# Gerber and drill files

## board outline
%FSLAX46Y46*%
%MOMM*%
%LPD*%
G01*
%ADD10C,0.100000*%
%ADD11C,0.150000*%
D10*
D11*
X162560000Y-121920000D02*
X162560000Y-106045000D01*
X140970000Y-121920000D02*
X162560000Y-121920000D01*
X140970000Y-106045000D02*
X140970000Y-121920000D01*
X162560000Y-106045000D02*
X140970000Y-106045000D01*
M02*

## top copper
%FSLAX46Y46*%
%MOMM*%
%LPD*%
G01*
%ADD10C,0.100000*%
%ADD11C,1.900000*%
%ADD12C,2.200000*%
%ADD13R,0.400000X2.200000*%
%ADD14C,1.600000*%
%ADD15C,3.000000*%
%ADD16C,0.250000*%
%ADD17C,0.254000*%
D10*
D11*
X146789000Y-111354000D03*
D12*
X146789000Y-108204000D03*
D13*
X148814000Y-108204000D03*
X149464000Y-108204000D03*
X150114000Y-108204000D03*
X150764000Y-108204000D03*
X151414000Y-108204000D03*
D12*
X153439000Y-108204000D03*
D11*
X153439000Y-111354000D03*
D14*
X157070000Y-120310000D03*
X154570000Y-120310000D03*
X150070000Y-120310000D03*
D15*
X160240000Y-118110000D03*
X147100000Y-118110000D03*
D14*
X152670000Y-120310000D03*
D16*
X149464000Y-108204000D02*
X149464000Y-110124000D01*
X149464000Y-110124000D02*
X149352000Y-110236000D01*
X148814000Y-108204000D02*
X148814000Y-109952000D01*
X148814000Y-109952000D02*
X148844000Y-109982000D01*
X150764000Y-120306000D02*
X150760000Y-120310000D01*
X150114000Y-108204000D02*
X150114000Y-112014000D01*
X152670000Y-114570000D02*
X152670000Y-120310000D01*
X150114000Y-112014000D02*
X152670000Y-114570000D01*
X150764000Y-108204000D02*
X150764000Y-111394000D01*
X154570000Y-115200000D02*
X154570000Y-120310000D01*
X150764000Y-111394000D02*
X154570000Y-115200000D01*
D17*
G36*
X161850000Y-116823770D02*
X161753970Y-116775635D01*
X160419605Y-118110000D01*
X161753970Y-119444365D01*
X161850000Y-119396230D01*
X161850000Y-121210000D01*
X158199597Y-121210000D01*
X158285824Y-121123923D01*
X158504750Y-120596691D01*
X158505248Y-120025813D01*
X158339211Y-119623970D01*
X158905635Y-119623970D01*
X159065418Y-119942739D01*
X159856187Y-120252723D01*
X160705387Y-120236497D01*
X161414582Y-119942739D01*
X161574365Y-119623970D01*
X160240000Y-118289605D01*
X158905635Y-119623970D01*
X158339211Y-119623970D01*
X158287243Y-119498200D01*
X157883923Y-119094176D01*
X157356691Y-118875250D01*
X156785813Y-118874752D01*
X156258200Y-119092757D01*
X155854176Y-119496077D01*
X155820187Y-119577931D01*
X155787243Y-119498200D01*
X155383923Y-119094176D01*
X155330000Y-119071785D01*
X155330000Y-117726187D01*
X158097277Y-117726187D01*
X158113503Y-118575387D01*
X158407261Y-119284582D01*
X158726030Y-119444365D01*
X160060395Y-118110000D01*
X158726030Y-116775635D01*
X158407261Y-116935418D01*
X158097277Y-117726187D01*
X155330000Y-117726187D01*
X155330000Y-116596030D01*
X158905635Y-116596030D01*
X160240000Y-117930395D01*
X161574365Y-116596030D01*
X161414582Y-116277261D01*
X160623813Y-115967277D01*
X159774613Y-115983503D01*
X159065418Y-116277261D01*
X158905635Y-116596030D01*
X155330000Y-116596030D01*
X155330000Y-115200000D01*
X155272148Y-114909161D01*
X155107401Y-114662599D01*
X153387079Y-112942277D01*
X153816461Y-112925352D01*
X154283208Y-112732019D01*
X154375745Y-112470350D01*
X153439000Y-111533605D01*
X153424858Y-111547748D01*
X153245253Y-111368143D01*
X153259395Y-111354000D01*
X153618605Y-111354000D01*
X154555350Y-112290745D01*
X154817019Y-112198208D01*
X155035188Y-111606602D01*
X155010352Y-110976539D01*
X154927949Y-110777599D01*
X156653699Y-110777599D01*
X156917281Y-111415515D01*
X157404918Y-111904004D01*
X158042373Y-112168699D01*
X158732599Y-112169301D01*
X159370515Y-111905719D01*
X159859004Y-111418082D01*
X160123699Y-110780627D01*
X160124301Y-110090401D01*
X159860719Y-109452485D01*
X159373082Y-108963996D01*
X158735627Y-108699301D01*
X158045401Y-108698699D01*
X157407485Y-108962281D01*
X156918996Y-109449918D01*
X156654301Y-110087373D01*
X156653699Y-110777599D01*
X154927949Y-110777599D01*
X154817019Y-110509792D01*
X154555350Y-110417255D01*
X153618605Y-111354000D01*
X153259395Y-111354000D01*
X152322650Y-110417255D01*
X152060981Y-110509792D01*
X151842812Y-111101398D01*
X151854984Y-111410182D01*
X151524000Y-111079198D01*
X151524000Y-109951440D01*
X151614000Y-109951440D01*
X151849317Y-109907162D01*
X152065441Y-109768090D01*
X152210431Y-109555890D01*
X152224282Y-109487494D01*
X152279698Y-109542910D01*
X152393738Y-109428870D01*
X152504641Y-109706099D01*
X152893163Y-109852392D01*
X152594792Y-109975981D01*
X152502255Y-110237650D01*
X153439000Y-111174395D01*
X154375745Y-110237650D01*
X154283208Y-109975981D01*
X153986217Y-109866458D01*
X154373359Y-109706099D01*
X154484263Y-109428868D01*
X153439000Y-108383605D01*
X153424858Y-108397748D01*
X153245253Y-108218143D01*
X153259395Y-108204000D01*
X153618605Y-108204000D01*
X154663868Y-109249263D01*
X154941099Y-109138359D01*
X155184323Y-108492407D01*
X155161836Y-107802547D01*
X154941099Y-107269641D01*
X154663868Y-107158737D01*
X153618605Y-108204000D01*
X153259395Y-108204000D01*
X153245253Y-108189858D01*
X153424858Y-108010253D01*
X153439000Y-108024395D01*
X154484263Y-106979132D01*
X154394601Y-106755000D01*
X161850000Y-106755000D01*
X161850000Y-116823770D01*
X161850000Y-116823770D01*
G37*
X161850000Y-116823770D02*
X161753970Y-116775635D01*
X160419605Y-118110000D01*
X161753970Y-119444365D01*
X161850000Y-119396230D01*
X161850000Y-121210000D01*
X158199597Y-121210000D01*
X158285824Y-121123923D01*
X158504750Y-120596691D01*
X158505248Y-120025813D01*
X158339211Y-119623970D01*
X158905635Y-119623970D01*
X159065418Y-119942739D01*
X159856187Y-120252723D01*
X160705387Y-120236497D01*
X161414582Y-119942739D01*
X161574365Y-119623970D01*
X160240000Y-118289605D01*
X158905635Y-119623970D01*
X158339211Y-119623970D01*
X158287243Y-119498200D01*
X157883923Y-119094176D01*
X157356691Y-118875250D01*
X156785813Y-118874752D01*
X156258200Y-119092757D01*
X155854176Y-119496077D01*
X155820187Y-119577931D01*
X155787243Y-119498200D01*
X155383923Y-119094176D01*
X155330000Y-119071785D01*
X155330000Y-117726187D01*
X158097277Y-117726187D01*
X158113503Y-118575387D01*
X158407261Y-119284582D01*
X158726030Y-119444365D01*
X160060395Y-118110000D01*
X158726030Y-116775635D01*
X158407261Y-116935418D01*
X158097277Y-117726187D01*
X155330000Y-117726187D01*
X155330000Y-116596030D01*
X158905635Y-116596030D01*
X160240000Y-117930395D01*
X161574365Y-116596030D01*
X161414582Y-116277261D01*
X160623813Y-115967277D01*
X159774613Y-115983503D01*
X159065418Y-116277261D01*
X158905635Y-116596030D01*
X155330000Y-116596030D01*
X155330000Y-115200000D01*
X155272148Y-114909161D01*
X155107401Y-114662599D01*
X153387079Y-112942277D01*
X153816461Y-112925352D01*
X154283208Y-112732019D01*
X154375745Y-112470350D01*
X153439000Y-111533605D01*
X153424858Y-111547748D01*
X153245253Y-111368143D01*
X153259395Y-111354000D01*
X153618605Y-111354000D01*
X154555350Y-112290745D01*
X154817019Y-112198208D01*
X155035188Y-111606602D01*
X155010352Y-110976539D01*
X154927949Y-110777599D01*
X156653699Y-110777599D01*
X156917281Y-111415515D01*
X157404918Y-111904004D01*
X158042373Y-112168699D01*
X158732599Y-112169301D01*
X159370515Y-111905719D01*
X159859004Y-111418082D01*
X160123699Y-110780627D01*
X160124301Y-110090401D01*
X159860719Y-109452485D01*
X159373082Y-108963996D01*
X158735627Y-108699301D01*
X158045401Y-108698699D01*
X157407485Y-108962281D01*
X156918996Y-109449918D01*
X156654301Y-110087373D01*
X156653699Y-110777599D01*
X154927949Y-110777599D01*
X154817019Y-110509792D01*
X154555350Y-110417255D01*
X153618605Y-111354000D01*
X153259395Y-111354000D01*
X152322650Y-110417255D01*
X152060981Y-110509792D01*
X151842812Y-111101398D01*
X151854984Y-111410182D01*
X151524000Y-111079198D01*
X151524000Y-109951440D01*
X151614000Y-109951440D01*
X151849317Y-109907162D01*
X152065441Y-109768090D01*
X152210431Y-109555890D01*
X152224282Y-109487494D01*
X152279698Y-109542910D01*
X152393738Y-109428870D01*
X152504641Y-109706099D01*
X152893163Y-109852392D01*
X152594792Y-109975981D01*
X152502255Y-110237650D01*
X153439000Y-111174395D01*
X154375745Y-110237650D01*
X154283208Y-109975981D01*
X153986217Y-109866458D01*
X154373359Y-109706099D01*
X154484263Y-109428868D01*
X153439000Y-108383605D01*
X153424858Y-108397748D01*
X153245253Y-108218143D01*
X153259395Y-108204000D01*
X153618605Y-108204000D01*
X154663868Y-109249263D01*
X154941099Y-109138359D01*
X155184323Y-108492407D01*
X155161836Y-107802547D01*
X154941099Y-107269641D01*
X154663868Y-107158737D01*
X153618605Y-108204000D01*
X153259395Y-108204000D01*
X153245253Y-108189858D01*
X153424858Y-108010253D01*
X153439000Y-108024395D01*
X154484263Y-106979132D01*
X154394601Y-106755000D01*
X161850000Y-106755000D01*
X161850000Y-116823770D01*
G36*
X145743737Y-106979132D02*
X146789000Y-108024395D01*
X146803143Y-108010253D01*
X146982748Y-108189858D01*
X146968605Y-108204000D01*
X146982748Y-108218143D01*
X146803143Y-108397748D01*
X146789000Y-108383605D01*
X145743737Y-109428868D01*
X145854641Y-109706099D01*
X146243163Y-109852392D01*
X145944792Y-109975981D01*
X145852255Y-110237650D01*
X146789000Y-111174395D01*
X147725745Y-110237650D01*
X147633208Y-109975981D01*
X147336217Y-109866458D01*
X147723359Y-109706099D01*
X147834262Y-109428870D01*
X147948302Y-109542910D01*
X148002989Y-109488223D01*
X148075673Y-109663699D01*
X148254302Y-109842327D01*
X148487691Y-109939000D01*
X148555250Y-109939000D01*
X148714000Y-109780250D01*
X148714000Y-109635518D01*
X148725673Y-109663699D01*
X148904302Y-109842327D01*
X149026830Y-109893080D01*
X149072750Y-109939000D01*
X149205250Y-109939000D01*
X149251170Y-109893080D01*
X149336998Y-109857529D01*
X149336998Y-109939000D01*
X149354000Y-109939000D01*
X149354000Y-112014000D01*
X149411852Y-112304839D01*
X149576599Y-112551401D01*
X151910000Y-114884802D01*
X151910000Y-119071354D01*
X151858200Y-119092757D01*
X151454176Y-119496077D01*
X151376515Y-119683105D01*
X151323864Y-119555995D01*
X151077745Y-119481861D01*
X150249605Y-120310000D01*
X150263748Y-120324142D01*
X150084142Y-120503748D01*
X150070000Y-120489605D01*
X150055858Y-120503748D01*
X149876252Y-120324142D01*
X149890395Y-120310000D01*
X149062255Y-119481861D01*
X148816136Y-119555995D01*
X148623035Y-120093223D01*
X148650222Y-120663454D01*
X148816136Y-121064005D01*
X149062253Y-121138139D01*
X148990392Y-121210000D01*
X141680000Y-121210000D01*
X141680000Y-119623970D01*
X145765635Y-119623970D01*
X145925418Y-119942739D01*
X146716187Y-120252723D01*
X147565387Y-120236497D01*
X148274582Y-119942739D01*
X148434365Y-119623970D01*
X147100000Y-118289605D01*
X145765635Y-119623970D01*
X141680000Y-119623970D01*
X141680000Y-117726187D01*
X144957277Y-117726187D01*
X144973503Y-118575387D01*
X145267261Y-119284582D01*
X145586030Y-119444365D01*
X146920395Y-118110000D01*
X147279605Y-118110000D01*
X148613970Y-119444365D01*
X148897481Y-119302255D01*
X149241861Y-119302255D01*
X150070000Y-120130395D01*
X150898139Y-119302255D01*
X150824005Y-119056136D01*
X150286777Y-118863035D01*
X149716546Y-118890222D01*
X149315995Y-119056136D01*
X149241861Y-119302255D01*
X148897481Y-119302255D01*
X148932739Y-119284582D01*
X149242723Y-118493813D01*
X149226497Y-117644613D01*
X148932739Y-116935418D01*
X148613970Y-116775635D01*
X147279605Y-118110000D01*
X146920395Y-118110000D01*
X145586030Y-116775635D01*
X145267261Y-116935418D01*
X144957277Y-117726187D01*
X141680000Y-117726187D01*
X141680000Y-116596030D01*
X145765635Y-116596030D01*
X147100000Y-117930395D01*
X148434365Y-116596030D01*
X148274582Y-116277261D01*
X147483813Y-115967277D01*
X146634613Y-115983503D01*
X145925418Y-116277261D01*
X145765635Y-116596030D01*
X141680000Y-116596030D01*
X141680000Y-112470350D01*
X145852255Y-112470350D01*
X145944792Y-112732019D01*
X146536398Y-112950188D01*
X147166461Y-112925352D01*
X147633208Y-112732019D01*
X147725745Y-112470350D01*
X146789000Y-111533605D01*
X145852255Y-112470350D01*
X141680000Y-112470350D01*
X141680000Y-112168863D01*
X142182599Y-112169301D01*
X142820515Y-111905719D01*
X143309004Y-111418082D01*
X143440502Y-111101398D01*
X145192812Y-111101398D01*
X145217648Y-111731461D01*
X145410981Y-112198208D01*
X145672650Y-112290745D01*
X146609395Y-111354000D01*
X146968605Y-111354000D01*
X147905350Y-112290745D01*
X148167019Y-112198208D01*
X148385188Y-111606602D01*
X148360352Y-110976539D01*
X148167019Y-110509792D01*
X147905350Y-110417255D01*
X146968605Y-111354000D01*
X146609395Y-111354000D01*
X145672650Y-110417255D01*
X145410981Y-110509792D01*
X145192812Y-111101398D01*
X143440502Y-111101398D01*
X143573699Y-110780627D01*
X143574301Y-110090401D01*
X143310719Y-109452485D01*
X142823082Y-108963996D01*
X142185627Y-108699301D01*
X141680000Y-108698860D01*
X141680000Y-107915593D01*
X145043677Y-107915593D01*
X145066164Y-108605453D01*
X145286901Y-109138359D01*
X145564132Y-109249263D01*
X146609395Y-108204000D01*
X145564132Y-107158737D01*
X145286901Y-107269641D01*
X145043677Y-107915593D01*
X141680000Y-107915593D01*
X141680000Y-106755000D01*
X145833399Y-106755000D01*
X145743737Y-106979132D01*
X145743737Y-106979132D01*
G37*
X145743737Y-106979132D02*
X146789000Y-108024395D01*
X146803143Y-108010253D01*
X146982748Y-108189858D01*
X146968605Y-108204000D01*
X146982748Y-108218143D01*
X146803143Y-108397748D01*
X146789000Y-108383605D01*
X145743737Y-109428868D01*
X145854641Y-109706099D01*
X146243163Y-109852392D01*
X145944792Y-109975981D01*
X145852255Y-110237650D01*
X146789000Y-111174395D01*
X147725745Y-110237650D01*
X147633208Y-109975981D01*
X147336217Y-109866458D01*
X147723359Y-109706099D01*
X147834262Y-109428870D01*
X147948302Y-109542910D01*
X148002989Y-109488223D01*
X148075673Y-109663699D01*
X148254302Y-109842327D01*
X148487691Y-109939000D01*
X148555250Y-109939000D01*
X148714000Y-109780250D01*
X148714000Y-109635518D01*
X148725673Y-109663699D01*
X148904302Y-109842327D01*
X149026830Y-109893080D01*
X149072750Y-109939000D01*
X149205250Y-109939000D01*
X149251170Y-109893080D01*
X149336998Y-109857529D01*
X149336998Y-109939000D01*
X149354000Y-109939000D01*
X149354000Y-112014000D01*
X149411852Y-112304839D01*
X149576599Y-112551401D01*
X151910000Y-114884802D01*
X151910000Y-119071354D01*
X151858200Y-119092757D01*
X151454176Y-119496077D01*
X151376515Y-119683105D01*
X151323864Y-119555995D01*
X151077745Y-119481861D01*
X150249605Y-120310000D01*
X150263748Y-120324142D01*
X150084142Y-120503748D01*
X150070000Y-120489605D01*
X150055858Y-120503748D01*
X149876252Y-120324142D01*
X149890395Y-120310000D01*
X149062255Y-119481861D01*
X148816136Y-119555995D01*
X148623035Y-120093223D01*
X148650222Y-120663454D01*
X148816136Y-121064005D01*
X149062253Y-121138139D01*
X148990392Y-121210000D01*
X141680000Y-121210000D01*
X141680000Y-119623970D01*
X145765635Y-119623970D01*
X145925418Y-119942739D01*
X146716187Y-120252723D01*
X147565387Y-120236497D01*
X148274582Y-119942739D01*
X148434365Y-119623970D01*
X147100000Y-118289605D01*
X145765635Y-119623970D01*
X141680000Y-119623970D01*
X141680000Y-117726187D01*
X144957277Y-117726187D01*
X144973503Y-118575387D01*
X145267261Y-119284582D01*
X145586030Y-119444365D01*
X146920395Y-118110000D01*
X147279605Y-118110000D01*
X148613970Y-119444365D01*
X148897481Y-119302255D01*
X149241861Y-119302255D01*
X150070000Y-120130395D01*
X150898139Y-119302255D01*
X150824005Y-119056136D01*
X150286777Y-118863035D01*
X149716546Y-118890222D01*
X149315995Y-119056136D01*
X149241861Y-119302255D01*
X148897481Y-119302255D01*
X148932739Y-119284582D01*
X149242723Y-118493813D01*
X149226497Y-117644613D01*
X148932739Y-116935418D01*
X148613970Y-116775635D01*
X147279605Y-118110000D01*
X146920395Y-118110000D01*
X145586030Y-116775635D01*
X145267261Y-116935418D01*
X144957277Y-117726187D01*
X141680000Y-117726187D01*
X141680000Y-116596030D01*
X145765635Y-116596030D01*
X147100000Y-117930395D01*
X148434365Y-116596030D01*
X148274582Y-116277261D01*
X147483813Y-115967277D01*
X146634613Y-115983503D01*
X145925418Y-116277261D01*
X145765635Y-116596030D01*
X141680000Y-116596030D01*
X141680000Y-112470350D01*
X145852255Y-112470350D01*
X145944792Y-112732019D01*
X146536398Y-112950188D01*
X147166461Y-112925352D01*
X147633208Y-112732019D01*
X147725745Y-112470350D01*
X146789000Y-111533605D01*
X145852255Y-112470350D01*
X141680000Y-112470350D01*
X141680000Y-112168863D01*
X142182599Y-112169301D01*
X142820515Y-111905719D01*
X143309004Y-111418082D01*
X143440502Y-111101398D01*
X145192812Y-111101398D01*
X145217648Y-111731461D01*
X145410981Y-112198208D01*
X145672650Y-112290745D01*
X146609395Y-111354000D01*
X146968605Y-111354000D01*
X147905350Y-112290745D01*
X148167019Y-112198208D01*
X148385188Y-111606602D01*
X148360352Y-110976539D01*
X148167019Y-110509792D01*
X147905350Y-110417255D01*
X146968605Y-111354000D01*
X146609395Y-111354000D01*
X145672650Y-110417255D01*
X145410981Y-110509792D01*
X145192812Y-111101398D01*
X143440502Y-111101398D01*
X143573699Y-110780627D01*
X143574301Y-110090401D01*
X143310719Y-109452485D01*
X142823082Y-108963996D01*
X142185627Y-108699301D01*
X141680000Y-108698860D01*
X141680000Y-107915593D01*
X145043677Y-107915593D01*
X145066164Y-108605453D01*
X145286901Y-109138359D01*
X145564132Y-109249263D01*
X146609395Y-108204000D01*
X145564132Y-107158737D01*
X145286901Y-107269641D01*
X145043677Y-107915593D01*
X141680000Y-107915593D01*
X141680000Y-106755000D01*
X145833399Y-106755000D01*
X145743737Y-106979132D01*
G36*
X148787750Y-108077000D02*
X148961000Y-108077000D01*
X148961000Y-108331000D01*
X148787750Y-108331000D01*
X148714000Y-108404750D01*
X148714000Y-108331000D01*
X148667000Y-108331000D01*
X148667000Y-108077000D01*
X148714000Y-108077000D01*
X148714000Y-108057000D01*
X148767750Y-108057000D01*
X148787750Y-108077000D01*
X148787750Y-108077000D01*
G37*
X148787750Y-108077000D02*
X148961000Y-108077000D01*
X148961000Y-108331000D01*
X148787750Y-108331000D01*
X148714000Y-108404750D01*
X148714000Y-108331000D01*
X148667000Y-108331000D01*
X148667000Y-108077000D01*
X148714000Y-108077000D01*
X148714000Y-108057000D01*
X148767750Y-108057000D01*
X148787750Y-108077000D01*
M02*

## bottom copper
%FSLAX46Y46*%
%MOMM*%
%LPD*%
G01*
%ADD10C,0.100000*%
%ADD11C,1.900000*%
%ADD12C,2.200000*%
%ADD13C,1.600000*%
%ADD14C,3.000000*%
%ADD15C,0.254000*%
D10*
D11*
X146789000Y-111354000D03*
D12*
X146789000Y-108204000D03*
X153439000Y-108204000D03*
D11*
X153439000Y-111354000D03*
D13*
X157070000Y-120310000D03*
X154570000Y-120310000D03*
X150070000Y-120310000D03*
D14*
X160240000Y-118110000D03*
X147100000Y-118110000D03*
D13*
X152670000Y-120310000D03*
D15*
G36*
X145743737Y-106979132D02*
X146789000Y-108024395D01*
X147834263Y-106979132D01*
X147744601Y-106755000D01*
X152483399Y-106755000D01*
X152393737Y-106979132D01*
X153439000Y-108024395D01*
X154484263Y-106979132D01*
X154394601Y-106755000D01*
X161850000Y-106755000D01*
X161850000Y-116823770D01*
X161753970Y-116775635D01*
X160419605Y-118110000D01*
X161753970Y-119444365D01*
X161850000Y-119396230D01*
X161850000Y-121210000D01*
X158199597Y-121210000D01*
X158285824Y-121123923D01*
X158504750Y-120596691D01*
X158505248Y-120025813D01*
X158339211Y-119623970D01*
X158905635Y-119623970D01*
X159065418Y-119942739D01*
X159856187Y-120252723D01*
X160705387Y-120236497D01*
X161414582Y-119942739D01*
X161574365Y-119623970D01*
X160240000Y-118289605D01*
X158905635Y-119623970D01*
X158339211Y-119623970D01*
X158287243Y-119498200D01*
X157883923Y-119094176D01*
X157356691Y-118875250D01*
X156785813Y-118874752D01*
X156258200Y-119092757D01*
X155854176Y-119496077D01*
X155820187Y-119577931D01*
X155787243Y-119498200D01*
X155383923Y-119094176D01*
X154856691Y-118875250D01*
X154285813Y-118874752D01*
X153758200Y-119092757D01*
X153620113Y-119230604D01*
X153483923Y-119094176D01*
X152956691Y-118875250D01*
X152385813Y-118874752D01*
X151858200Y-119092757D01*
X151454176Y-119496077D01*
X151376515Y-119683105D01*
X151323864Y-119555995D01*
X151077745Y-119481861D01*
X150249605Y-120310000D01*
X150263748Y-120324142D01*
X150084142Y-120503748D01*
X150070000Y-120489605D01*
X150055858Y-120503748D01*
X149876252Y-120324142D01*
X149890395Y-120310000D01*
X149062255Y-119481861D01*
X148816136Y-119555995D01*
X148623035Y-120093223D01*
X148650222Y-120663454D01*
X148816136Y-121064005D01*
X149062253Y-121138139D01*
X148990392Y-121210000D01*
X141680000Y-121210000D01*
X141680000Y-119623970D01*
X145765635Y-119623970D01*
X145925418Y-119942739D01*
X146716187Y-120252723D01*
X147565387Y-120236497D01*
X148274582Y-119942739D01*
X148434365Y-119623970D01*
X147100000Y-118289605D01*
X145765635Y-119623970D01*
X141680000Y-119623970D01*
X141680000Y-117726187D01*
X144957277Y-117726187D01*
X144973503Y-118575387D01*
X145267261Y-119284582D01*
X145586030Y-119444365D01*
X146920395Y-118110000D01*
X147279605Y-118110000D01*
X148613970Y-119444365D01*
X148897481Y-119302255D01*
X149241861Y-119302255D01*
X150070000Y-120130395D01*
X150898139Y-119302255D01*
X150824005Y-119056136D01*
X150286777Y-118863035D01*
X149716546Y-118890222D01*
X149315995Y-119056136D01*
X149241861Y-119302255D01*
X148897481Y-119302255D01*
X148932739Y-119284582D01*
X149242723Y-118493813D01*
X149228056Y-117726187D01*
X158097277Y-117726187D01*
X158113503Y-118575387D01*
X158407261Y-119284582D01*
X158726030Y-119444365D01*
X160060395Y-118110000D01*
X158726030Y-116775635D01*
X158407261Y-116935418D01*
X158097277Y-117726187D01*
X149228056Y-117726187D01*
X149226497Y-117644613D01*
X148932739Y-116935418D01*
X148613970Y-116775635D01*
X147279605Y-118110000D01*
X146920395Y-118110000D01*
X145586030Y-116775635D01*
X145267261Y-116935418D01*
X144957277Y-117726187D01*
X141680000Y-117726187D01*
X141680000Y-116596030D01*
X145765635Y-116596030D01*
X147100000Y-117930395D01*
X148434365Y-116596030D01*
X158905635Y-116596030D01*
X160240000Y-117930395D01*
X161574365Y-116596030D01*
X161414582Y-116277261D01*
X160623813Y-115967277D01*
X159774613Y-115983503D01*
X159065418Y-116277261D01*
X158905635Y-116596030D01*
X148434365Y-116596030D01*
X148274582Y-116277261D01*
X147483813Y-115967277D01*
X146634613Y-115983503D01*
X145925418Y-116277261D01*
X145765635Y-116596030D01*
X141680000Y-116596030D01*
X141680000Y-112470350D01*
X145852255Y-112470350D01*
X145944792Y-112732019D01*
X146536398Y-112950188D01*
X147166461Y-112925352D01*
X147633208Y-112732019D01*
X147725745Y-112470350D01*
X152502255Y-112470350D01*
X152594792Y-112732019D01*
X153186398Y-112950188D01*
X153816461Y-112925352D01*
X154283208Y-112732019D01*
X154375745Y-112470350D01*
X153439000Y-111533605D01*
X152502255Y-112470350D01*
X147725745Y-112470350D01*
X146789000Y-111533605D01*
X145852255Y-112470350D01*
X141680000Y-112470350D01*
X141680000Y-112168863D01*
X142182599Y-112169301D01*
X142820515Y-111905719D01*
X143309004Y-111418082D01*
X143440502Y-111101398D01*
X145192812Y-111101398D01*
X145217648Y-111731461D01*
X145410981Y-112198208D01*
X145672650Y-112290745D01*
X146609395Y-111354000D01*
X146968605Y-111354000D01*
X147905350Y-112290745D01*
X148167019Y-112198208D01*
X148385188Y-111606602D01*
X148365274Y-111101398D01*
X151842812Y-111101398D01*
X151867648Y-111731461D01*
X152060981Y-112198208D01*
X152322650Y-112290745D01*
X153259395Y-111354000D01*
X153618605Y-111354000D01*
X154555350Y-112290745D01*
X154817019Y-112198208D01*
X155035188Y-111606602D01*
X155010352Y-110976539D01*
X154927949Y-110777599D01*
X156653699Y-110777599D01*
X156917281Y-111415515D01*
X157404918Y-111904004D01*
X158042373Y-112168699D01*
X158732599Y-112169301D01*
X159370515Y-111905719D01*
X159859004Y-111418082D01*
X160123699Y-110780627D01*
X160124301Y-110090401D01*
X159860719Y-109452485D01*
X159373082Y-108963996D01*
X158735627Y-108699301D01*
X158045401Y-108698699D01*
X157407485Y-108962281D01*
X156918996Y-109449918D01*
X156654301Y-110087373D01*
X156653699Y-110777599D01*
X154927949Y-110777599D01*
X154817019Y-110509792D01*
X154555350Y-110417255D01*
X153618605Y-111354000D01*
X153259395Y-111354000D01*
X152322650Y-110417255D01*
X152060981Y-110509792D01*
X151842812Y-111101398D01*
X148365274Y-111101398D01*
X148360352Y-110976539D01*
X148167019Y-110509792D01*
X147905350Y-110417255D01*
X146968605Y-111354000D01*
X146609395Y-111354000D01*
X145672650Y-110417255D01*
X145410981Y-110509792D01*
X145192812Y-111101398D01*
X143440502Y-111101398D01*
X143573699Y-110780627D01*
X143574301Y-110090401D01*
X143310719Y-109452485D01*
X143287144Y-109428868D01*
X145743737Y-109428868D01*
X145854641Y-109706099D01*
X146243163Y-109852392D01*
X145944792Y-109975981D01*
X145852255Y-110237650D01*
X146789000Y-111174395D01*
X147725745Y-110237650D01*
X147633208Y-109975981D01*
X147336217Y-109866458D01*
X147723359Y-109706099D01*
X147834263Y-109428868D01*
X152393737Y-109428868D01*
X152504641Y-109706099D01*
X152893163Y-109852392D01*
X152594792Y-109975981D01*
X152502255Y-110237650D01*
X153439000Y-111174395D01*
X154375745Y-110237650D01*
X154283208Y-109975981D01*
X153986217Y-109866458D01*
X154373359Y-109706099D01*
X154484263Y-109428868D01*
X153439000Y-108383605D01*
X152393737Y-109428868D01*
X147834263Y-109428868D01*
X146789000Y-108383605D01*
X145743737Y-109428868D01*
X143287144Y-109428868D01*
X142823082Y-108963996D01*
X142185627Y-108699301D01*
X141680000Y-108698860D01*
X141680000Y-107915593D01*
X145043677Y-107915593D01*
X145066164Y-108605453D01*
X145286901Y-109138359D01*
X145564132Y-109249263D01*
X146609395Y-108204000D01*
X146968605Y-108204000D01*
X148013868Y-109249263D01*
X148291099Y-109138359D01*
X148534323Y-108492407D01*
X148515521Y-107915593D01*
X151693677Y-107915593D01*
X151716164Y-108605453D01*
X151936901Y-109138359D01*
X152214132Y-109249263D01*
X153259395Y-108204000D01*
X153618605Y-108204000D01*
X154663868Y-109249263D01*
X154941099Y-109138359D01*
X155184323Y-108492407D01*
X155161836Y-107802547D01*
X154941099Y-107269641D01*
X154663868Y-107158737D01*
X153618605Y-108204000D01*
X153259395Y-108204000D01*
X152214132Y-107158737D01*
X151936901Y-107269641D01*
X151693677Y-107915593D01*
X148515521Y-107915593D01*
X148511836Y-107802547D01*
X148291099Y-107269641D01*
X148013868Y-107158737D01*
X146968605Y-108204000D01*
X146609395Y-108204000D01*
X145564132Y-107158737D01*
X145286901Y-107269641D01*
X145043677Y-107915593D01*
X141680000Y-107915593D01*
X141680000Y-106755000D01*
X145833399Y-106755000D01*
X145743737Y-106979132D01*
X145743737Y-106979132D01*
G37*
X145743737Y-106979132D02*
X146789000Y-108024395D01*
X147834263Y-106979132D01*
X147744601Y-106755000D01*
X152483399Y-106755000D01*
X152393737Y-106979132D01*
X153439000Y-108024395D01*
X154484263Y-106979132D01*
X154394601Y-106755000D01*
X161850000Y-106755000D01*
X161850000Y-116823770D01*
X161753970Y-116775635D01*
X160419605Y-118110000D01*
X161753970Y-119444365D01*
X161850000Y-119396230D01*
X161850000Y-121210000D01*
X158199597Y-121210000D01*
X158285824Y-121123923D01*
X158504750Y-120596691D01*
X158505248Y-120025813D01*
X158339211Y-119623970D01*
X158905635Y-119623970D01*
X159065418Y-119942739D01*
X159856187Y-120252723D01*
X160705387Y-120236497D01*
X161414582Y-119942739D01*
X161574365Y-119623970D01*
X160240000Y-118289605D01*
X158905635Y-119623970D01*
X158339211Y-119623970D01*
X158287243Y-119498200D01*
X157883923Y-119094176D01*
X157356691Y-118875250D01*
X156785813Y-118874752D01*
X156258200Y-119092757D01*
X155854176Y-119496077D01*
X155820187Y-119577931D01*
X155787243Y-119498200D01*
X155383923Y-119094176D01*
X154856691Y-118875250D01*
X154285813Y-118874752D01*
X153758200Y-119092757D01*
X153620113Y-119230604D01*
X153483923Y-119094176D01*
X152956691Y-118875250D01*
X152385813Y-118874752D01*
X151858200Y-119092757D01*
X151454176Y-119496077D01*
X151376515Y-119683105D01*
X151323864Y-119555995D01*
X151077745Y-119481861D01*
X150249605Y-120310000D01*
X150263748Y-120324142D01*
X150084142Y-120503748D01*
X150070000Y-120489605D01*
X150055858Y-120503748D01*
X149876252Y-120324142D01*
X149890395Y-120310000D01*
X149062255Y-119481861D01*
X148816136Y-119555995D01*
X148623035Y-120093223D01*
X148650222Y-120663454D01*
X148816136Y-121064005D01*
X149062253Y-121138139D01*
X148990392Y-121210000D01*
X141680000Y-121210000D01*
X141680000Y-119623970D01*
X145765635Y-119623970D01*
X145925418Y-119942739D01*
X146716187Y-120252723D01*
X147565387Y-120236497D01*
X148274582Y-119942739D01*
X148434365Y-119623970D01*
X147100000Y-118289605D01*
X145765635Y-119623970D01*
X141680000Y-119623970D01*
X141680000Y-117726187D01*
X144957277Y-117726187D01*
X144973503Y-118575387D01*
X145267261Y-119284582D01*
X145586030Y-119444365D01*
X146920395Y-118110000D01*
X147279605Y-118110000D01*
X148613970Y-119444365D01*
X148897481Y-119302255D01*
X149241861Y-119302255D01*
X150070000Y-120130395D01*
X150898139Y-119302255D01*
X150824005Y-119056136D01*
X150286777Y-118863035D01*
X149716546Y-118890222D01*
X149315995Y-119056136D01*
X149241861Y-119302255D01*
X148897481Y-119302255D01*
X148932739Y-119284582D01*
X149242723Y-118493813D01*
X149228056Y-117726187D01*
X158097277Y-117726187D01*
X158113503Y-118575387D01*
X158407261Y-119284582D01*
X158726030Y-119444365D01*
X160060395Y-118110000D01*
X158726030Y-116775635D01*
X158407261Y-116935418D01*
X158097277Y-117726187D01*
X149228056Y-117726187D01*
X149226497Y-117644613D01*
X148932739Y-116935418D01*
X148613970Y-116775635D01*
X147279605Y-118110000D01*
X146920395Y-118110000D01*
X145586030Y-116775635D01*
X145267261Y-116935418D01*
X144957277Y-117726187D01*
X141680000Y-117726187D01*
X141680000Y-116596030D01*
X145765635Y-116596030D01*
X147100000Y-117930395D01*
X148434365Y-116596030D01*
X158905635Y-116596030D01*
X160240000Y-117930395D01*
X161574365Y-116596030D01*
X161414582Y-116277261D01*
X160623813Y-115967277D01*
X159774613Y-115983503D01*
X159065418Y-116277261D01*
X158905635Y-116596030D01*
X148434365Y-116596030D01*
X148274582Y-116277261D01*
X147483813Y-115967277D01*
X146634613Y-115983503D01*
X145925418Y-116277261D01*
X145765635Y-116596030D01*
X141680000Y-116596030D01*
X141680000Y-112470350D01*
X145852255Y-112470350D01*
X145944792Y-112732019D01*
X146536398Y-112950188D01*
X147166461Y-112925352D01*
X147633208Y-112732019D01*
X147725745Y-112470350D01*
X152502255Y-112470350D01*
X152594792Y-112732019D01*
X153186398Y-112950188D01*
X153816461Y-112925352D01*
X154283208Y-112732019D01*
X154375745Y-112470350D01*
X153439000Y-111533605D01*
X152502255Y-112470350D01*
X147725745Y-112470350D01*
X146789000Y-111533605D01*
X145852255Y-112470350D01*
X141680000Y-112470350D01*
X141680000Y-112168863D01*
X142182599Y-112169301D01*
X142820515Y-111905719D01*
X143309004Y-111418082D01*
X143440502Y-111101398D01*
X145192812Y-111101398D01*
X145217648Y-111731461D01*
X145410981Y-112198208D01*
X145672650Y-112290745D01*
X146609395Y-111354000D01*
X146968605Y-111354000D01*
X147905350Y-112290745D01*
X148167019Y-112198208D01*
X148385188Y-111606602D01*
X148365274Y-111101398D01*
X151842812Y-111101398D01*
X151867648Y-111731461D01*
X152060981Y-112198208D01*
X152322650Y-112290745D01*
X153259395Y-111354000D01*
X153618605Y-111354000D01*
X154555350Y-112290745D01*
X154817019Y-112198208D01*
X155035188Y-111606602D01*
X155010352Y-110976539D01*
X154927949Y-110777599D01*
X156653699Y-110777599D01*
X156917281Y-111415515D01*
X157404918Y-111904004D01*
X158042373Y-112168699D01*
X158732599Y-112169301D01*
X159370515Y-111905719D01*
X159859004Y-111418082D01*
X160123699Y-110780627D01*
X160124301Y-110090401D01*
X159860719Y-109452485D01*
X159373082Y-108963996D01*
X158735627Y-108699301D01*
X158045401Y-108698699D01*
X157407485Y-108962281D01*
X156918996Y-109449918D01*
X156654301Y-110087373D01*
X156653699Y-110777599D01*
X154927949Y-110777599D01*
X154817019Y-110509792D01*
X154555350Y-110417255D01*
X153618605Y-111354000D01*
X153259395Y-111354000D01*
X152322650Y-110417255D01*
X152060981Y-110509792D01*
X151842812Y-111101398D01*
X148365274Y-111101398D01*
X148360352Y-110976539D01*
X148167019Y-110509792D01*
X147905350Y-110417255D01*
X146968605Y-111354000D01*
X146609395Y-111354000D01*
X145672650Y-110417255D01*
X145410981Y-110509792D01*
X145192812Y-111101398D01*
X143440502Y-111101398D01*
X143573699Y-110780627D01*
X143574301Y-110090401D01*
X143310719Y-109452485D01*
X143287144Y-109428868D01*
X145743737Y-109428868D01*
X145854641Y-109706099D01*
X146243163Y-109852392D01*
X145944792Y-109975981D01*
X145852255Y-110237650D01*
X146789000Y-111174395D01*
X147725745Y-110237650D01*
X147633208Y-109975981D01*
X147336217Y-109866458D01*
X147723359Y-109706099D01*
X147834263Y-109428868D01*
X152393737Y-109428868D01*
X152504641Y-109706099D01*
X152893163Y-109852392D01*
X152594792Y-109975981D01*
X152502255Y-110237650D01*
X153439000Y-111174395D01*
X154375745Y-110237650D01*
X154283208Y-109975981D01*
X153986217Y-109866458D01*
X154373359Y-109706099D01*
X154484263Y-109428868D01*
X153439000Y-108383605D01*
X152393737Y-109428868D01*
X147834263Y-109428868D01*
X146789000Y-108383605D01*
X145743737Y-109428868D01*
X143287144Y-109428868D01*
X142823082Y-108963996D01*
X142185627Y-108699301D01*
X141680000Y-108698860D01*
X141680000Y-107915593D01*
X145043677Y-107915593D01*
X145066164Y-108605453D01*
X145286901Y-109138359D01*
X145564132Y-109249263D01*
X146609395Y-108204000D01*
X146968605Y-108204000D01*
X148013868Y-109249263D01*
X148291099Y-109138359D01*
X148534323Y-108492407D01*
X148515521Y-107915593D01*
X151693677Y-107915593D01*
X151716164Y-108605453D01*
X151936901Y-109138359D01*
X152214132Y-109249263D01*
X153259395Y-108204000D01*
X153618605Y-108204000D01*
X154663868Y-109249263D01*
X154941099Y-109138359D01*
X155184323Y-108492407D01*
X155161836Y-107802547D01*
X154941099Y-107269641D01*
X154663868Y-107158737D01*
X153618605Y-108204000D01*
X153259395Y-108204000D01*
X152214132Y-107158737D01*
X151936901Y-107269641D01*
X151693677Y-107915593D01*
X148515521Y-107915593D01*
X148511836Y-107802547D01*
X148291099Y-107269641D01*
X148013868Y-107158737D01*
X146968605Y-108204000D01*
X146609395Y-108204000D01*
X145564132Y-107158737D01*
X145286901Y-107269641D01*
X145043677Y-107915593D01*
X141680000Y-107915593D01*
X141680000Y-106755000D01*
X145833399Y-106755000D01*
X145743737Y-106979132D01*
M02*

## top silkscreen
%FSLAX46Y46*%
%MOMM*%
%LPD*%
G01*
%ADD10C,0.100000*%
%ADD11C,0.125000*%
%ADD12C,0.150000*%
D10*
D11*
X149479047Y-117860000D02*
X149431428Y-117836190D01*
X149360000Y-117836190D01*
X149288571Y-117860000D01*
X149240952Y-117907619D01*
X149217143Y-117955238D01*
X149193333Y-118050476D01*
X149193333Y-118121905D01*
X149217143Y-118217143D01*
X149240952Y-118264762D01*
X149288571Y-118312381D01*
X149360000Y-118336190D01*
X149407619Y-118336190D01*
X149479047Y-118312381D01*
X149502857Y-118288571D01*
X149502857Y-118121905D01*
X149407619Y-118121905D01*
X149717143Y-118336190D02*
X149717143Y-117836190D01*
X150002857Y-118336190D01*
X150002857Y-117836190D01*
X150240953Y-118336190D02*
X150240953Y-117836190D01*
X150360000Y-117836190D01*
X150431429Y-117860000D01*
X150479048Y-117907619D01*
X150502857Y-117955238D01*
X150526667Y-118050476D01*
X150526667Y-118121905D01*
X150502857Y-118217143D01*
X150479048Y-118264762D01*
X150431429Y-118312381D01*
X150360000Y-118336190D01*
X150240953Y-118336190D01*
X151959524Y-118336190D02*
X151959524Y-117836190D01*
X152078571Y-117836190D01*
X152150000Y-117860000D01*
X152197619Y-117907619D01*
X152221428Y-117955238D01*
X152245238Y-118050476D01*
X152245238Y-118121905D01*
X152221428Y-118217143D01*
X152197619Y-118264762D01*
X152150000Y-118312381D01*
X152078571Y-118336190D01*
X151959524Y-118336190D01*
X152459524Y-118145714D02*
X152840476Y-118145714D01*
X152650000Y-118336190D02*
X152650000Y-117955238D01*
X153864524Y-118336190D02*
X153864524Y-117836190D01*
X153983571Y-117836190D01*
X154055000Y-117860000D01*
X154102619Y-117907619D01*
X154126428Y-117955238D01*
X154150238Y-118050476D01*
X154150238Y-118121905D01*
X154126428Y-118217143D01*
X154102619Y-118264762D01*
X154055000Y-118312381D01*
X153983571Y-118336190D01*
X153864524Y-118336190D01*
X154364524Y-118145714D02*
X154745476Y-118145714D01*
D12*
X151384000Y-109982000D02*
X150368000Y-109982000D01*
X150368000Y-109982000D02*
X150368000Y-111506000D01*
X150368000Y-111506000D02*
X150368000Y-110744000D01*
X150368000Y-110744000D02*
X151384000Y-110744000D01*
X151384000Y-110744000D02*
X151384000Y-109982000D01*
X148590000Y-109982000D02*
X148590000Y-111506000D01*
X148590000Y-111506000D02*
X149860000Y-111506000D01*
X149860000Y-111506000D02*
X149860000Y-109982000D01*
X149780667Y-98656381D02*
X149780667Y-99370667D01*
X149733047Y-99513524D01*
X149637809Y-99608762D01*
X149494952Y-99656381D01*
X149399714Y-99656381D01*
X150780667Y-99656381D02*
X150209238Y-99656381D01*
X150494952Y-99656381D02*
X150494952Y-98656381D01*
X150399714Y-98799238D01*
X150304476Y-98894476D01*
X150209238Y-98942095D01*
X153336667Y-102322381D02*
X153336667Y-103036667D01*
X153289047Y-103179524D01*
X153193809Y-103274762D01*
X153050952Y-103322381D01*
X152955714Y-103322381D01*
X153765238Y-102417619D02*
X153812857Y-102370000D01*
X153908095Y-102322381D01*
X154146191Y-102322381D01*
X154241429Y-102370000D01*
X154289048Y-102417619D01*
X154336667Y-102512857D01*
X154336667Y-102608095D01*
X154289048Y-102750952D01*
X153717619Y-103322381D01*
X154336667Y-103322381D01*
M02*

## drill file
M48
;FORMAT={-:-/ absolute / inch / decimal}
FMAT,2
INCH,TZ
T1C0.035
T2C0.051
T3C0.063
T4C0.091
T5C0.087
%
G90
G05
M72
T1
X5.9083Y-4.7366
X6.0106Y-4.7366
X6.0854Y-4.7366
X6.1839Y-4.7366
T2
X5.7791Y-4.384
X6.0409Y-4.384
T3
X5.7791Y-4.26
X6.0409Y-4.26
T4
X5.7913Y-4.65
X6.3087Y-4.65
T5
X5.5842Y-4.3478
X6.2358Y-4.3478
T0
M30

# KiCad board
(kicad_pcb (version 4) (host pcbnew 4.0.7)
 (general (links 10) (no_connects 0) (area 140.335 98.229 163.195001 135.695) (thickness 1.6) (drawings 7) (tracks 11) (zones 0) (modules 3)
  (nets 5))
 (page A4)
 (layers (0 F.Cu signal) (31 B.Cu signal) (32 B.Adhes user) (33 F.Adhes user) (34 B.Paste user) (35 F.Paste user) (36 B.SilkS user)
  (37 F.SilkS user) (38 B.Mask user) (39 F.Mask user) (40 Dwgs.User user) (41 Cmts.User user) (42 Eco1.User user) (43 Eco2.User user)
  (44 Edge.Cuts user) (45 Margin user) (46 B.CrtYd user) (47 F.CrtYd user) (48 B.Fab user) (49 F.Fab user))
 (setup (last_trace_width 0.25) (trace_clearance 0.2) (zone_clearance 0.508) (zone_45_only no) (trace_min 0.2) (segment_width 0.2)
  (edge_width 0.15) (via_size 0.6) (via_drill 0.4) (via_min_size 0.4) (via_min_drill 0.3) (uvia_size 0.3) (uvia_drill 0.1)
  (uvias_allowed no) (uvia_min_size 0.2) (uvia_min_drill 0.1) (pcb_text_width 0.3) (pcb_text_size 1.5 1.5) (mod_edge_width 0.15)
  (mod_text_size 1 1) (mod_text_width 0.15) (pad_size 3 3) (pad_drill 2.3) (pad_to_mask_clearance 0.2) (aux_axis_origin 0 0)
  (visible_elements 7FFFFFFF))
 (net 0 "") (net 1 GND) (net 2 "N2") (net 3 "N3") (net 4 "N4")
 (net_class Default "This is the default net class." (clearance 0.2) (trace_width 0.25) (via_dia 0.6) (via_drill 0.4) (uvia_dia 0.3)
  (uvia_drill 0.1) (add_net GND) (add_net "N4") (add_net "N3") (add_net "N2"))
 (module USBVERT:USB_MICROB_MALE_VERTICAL (layer F.Cu) (at 150.114 108.204 180)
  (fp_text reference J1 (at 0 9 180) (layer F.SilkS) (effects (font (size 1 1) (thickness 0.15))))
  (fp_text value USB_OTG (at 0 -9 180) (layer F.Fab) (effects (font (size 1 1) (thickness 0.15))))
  (fp_line (start -1.27 -1.778) (end -0.254 -1.778) (layer F.SilkS) (width 0.15))
  (fp_line (start -0.254 -1.778) (end -0.254 -3.302) (layer F.SilkS) (width 0.15))
  (fp_line (start -0.254 -3.302) (end -0.254 -2.54) (layer F.SilkS) (width 0.15))
  (fp_line (start -0.254 -2.54) (end -1.27 -2.54) (layer F.SilkS) (width 0.15))
  (fp_line (start -1.27 -2.54) (end -1.27 -1.778) (layer F.SilkS) (width 0.15))
  (fp_line (start 1.524 -1.778) (end 1.524 -3.302) (layer F.SilkS) (width 0.15))
  (fp_line (start 1.524 -3.302) (end 0.254 -3.302) (layer F.SilkS) (width 0.15))
  (fp_line (start 0.254 -3.302) (end 0.254 -1.778) (layer F.SilkS) (width 0.15))
  (pad "" np_thru_hole circle (at 8.275 -2.23 180) (size 2.2 2.2) (drill 2.2) (layers *.Cu *.Mask))
  (pad 6 thru_hole circle (at 3.325 -3.15 180) (size 1.9 1.9) (drill 1.3) (layers *.Cu *.Mask) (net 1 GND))
  (pad 6 thru_hole circle (at 3.325 0 180) (size 2.2 2.2) (drill 1.6) (layers *.Cu *.Mask) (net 1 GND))
  (pad 5 smd rect (at 1.3 0 180) (size 0.4 2.2) (layers F.Cu F.Paste F.Mask) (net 1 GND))
  (pad 4 smd rect (at 0.65 0 180) (size 0.4 2.2) (layers F.Cu F.Paste F.Mask) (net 1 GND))
  (pad 3 smd rect (at 0 0 180) (size 0.4 2.2) (layers F.Cu F.Paste F.Mask) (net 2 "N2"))
  (pad 2 smd rect (at -0.65 0 180) (size 0.4 2.2) (layers F.Cu F.Paste F.Mask) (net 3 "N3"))
  (pad 1 smd rect (at -1.3 0 180) (size 0.4 2.2) (layers F.Cu F.Paste F.Mask) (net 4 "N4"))
  (pad 6 thru_hole circle (at -3.325 0 180) (size 2.2 2.2) (drill 1.6) (layers *.Cu *.Mask) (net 1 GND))
  (pad 6 thru_hole circle (at -3.325 -3.15 180) (size 1.9 1.9) (drill 1.3) (layers *.Cu *.Mask) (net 1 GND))
  (pad "" np_thru_hole circle (at -8.275 -2.23 180) (size 2.2 2.2) (drill 2.2) (layers *.Cu *.Mask)))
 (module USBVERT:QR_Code (layer B.Cu) (at 153.67 115.57)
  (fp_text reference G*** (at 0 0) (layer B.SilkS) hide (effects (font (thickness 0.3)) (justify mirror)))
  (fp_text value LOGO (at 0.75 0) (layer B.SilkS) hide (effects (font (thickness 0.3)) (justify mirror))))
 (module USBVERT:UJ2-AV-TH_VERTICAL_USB (layer F.Cu) (at 153.67 118.11 180)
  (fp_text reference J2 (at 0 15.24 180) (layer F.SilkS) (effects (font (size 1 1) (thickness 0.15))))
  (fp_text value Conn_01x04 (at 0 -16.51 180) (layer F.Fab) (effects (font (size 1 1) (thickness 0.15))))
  (pad 1 thru_hole circle (at -3.4 -2.2 180) (size 1.6 1.6) (drill 0.9) (layers *.Cu *.Mask))
  (pad 2 thru_hole circle (at -0.9 -2.2 180) (size 1.6 1.6) (drill 0.9) (layers *.Cu *.Mask) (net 3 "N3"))
  (pad 4 thru_hole circle (at 3.6 -2.2 180) (size 1.6 1.6) (drill 0.9) (layers *.Cu *.Mask) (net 1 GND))
  (pad 5 thru_hole circle (at -6.57 0 180) (size 3 3) (drill 2.3) (layers *.Cu *.Mask) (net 1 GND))
  (pad 5 thru_hole circle (at 6.57 0 180) (size 3 3) (drill 2.3) (layers *.Cu *.Mask) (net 1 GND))
  (pad 3 thru_hole circle (at 1 -2.2 180) (size 1.6 1.6) (drill 0.9) (layers *.Cu *.Mask) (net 2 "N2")))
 (gr_line (start 162.56 121.92) (end 162.56 106.045) (angle 90) (layer Edge.Cuts) (width 0.15))
 (gr_line (start 140.97 121.92) (end 162.56 121.92) (angle 90) (layer Edge.Cuts) (width 0.15))
 (gr_line (start 140.97 106.045) (end 140.97 121.92) (angle 90) (layer Edge.Cuts) (width 0.15))
 (gr_line (start 162.56 106.045) (end 140.97 106.045) (angle 90) (layer Edge.Cuts) (width 0.15))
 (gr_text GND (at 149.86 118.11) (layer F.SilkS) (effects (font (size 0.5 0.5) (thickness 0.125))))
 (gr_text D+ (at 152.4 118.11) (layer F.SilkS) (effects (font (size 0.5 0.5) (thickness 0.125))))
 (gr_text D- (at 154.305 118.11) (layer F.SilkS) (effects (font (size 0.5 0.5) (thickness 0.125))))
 (segment (start 149.464 108.204) (end 149.464 110.124) (width 0.25) (layer F.Cu) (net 1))
 (segment (start 149.464 110.124) (end 149.352 110.236) (width 0.25) (layer F.Cu) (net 1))
 (segment (start 148.814 108.204) (end 148.814 109.952) (width 0.25) (layer F.Cu) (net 1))
 (segment (start 148.814 109.952) (end 148.844 109.982) (width 0.25) (layer F.Cu) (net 1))
 (segment (start 150.764 120.306) (end 150.76 120.31) (width 0.25) (layer F.Cu) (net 1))
 (segment (start 150.114 108.204) (end 150.114 112.014) (width 0.25) (layer F.Cu) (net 2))
 (segment (start 152.67 114.57) (end 152.67 120.31) (width 0.25) (layer F.Cu) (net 2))
 (segment (start 150.114 112.014) (end 152.67 114.57) (width 0.25) (layer F.Cu) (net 2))
 (segment (start 150.764 108.204) (end 150.764 111.394) (width 0.25) (layer F.Cu) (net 3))
 (segment (start 154.57 115.2) (end 154.57 120.31) (width 0.25) (layer F.Cu) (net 3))
 (segment (start 150.764 111.394) (end 154.57 115.2) (width 0.25) (layer F.Cu) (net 3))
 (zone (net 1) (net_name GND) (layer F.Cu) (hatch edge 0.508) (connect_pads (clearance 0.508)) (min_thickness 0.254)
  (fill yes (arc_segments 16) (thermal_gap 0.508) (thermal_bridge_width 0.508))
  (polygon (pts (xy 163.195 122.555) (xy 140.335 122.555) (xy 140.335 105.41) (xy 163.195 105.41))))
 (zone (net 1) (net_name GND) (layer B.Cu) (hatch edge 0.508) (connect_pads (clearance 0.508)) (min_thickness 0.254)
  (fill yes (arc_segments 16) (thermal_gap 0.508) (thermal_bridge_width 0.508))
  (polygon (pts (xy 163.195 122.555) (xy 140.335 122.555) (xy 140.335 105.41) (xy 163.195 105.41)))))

